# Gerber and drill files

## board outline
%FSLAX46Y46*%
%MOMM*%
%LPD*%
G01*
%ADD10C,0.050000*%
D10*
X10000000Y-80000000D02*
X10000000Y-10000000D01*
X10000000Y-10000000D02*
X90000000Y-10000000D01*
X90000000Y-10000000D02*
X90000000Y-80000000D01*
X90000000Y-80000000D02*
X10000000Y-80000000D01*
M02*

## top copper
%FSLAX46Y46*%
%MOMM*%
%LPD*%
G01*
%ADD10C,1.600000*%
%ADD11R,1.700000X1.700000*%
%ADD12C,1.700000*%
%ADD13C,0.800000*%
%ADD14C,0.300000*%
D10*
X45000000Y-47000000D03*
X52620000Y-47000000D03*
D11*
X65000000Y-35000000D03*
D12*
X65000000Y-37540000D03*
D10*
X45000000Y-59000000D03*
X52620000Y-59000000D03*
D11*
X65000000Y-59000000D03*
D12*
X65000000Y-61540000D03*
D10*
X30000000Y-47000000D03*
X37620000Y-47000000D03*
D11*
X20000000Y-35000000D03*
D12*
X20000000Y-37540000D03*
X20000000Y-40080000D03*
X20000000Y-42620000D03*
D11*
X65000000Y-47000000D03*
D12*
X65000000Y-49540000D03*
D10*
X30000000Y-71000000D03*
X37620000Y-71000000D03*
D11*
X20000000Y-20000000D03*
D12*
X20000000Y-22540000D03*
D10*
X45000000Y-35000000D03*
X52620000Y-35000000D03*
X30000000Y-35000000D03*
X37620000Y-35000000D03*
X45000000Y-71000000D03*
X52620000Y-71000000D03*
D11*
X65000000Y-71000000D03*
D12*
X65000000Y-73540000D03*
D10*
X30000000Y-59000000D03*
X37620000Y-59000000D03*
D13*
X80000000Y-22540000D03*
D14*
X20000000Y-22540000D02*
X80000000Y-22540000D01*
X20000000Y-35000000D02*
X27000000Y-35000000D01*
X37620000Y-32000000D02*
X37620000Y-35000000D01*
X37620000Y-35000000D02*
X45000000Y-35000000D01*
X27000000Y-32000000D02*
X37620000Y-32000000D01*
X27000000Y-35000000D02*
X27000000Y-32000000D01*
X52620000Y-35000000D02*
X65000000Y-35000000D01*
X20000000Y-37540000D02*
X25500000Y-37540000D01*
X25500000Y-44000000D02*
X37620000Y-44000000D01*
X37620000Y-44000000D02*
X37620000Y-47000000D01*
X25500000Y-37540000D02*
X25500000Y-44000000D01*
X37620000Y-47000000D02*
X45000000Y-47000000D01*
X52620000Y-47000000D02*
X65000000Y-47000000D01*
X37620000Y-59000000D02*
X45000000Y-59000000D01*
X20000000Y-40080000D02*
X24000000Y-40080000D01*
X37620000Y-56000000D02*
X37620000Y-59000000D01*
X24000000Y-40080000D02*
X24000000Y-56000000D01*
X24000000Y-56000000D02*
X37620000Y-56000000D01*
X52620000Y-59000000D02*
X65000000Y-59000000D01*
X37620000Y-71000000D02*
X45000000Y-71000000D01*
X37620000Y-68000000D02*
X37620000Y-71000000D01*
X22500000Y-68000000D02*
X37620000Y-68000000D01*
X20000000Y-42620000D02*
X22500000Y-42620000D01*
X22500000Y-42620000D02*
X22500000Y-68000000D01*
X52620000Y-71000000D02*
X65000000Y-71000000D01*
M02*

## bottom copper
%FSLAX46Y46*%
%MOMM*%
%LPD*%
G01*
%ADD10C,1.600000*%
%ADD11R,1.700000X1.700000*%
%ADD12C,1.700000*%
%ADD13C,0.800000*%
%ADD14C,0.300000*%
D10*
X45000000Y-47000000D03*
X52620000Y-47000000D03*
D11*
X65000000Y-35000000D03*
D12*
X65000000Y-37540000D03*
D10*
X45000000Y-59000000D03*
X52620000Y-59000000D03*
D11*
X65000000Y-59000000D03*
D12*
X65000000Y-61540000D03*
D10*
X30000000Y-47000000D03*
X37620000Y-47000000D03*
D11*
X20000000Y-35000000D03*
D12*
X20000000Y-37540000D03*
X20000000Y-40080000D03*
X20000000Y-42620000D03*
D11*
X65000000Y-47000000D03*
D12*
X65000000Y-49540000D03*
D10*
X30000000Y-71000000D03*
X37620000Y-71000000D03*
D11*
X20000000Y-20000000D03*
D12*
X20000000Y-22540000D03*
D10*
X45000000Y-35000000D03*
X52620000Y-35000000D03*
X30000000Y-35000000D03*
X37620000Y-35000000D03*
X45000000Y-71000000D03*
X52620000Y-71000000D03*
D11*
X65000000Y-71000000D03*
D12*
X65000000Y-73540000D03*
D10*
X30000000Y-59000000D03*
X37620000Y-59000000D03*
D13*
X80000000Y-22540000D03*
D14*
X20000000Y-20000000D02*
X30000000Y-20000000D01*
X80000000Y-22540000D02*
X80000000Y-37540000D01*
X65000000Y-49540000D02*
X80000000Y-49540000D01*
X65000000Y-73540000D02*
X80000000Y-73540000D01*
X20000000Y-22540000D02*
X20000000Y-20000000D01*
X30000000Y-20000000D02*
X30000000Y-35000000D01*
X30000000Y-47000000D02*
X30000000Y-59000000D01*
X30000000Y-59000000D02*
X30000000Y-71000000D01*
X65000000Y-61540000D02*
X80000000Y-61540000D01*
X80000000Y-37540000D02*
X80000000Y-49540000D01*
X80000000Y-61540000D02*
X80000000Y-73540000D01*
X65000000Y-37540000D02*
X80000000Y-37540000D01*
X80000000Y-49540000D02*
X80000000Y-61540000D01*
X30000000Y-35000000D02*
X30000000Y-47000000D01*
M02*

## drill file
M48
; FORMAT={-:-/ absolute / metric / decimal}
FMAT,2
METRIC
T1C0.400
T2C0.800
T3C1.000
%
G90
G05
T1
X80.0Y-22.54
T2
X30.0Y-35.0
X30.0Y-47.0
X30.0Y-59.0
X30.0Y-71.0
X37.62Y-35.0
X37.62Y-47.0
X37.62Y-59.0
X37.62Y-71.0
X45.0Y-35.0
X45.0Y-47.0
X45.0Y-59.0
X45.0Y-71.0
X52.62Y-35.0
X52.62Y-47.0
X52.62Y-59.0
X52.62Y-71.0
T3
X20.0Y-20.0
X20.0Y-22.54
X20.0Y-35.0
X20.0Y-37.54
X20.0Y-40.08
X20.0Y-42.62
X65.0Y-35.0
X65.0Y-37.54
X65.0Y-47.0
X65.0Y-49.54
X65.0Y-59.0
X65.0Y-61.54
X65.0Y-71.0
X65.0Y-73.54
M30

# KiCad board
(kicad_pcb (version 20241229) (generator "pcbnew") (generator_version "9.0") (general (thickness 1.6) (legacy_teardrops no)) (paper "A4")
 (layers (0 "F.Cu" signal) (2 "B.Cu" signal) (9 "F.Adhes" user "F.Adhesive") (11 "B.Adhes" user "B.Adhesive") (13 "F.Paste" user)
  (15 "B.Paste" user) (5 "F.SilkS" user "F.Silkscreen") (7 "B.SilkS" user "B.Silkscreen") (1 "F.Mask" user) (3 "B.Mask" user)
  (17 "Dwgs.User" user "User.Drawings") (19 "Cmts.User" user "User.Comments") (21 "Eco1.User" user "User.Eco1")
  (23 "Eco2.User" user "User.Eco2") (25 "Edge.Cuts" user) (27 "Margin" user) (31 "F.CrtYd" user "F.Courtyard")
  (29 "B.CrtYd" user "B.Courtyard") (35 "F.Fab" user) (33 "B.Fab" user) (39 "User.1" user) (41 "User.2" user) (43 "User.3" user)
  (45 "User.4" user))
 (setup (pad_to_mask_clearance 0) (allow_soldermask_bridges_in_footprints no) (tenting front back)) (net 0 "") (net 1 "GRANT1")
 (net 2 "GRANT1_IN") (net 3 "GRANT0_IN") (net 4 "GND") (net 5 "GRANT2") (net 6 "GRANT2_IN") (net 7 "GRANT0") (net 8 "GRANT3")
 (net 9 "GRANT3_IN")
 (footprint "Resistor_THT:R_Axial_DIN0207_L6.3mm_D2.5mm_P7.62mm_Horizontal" (layer "F.Cu") (at 45 47)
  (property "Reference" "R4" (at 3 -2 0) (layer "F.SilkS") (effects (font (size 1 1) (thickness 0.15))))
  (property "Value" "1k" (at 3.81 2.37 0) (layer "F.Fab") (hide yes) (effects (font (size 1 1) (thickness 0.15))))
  (pad "1" thru_hole circle (at 0 0) (size 1.6 1.6) (drill 0.8) (layers "*.Cu" "*.Mask") (remove_unused_layers no) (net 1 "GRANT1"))
  (pad "2" thru_hole circle (at 7.62 0) (size 1.6 1.6) (drill 0.8) (layers "*.Cu" "*.Mask") (remove_unused_layers no) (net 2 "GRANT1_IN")))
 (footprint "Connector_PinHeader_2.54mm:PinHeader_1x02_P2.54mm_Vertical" (layer "F.Cu") (at 65 35)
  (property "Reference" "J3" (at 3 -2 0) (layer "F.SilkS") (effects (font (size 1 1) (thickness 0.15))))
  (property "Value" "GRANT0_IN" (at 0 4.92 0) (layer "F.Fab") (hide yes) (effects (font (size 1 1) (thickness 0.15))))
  (pad "1" thru_hole rect (at 0 0) (size 1.7 1.7) (drill 1) (layers "*.Cu" "*.Mask") (remove_unused_layers no) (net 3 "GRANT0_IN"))
  (pad "2" thru_hole circle (at 0 2.54) (size 1.7 1.7) (drill 1) (layers "*.Cu" "*.Mask") (remove_unused_layers no) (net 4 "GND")))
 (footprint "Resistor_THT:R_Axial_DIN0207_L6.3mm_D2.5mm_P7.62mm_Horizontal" (layer "F.Cu") (at 45 59)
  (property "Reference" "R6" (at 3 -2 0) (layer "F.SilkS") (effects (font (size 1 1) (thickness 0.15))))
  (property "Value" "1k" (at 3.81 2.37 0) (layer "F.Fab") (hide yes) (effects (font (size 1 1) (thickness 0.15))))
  (pad "1" thru_hole circle (at 0 0) (size 1.6 1.6) (drill 0.8) (layers "*.Cu" "*.Mask") (remove_unused_layers no) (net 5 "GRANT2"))
  (pad "2" thru_hole circle (at 7.62 0) (size 1.6 1.6) (drill 0.8) (layers "*.Cu" "*.Mask") (remove_unused_layers no) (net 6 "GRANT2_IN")))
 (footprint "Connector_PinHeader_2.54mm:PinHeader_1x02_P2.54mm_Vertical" (layer "F.Cu") (at 65 59)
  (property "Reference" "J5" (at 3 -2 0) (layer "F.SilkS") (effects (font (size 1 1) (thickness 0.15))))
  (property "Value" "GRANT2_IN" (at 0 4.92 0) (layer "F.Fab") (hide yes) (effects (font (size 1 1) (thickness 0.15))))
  (pad "1" thru_hole rect (at 0 0) (size 1.7 1.7) (drill 1) (layers "*.Cu" "*.Mask") (remove_unused_layers no) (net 6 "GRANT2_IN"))
  (pad "2" thru_hole circle (at 0 2.54) (size 1.7 1.7) (drill 1) (layers "*.Cu" "*.Mask") (remove_unused_layers no) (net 4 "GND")))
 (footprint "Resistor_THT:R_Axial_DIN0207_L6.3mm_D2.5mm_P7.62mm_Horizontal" (layer "F.Cu") (at 30 47)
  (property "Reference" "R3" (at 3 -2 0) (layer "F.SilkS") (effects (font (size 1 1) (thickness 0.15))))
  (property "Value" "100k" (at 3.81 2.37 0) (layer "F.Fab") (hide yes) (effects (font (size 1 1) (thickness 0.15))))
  (pad "1" thru_hole circle (at 0 0) (size 1.6 1.6) (drill 0.8) (layers "*.Cu" "*.Mask") (remove_unused_layers no) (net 4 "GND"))
  (pad "2" thru_hole circle (at 7.62 0) (size 1.6 1.6) (drill 0.8) (layers "*.Cu" "*.Mask") (remove_unused_layers no) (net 1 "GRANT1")))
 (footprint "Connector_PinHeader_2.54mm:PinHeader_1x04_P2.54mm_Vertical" (layer "F.Cu") (at 20 35)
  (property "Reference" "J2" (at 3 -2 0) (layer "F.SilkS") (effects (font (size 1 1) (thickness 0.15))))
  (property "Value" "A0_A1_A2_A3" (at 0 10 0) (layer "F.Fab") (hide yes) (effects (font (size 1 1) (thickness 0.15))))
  (pad "1" thru_hole rect (at 0 0) (size 1.7 1.7) (drill 1) (layers "*.Cu" "*.Mask") (remove_unused_layers no) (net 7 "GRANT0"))
  (pad "2" thru_hole circle (at 0 2.54) (size 1.7 1.7) (drill 1) (layers "*.Cu" "*.Mask") (remove_unused_layers no) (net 1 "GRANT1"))
  (pad "3" thru_hole circle (at 0 5.08) (size 1.7 1.7) (drill 1) (layers "*.Cu" "*.Mask") (remove_unused_layers no) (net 5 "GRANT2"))
  (pad "4" thru_hole circle (at 0 7.62) (size 1.7 1.7) (drill 1) (layers "*.Cu" "*.Mask") (remove_unused_layers no) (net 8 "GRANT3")))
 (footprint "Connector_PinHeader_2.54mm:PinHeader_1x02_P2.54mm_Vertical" (layer "F.Cu") (at 65 47)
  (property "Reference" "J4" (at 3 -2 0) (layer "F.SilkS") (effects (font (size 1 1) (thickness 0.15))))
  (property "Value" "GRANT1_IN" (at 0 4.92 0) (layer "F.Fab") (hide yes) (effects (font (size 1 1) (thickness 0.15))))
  (pad "1" thru_hole rect (at 0 0) (size 1.7 1.7) (drill 1) (layers "*.Cu" "*.Mask") (remove_unused_layers no) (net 2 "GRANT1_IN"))
  (pad "2" thru_hole circle (at 0 2.54) (size 1.7 1.7) (drill 1) (layers "*.Cu" "*.Mask") (remove_unused_layers no) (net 4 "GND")))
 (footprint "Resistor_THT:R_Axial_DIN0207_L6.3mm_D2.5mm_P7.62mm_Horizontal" (layer "F.Cu") (at 30 71)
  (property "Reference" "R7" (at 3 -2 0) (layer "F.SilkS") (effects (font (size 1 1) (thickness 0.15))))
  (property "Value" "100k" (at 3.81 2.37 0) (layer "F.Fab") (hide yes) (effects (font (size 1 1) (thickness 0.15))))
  (pad "1" thru_hole circle (at 0 0) (size 1.6 1.6) (drill 0.8) (layers "*.Cu" "*.Mask") (remove_unused_layers no) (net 4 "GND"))
  (pad "2" thru_hole circle (at 7.62 0) (size 1.6 1.6) (drill 0.8) (layers "*.Cu" "*.Mask") (remove_unused_layers no) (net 8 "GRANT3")))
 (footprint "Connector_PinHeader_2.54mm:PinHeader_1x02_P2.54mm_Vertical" (layer "F.Cu") (at 20 20)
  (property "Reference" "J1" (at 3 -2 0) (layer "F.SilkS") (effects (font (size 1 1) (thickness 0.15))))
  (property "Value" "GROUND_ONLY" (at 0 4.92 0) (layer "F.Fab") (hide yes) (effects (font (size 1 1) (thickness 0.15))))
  (pad "1" thru_hole rect (at 0 0) (size 1.7 1.7) (drill 1) (layers "*.Cu" "*.Mask") (remove_unused_layers no) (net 4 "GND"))
  (pad "2" thru_hole circle (at 0 2.54) (size 1.7 1.7) (drill 1) (layers "*.Cu" "*.Mask") (remove_unused_layers no) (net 4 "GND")))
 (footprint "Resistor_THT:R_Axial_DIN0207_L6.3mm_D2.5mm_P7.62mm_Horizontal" (layer "F.Cu") (at 45 35)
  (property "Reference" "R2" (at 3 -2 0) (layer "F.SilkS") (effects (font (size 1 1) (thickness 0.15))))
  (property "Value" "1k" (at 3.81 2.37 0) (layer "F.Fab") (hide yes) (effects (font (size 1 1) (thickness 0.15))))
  (pad "1" thru_hole circle (at 0 0) (size 1.6 1.6) (drill 0.8) (layers "*.Cu" "*.Mask") (remove_unused_layers no) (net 7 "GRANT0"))
  (pad "2" thru_hole circle (at 7.62 0) (size 1.6 1.6) (drill 0.8) (layers "*.Cu" "*.Mask") (remove_unused_layers no) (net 3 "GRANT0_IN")))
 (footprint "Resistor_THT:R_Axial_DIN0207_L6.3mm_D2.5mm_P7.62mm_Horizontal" (layer "F.Cu") (at 30 35)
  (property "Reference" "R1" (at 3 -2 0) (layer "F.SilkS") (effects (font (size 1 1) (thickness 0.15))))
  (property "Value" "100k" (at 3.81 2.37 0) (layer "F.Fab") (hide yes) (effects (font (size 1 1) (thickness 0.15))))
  (pad "1" thru_hole circle (at 0 0) (size 1.6 1.6) (drill 0.8) (layers "*.Cu" "*.Mask") (remove_unused_layers no) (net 4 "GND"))
  (pad "2" thru_hole circle (at 7.62 0) (size 1.6 1.6) (drill 0.8) (layers "*.Cu" "*.Mask") (remove_unused_layers no) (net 7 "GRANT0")))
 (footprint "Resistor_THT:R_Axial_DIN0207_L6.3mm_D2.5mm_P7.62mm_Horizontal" (layer "F.Cu") (at 45 71)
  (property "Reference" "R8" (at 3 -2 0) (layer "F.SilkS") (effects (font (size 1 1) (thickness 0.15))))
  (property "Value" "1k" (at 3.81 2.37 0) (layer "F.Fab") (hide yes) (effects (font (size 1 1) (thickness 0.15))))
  (pad "1" thru_hole circle (at 0 0) (size 1.6 1.6) (drill 0.8) (layers "*.Cu" "*.Mask") (remove_unused_layers no) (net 8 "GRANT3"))
  (pad "2" thru_hole circle (at 7.62 0) (size 1.6 1.6) (drill 0.8) (layers "*.Cu" "*.Mask") (remove_unused_layers no) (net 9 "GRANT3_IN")))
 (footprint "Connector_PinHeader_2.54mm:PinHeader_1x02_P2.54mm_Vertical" (layer "F.Cu") (at 65 71)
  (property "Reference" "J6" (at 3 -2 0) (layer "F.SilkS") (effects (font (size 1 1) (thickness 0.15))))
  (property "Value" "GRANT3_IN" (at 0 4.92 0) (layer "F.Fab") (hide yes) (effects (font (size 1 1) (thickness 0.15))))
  (pad "1" thru_hole rect (at 0 0) (size 1.7 1.7) (drill 1) (layers "*.Cu" "*.Mask") (remove_unused_layers no) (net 9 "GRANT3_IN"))
  (pad "2" thru_hole circle (at 0 2.54) (size 1.7 1.7) (drill 1) (layers "*.Cu" "*.Mask") (remove_unused_layers no) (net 4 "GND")))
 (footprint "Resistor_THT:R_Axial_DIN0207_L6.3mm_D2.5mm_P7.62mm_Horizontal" (layer "F.Cu") (at 30 59)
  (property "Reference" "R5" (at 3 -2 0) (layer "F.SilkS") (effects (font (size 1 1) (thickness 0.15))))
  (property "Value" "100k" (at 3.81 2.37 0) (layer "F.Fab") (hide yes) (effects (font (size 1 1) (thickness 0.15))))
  (pad "1" thru_hole circle (at 0 0) (size 1.6 1.6) (drill 0.8) (layers "*.Cu" "*.Mask") (remove_unused_layers no) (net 4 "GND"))
  (pad "2" thru_hole circle (at 7.62 0) (size 1.6 1.6) (drill 0.8) (layers "*.Cu" "*.Mask") (remove_unused_layers no) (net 5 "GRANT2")))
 (gr_line (start 10 80) (end 10 10) (stroke (width 0.05) (type default)) (layer "Edge.Cuts"))
 (gr_line (start 10 10) (end 90 10) (stroke (width 0.05) (type default)) (layer "Edge.Cuts"))
 (gr_line (start 90 10) (end 90 80) (stroke (width 0.05) (type default)) (layer "Edge.Cuts"))
 (gr_line (start 90 80) (end 10 80) (stroke (width 0.05) (type default)) (layer "Edge.Cuts"))
 (segment (start 20 22.54) (end 80 22.54) (width 0.3) (layer "F.Cu") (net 4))
 (via (at 80 22.54) (size 0.8) (drill 0.4) (layers "F.Cu" "B.Cu") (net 4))
 (segment (start 20 20) (end 30 20) (width 0.3) (layer "B.Cu") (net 4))
 (segment (start 80 22.54) (end 80 37.54) (width 0.3) (layer "B.Cu") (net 4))
 (segment (start 65 49.54) (end 80 49.54) (width 0.3) (layer "B.Cu") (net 4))
 (segment (start 65 73.54) (end 80 73.54) (width 0.3) (layer "B.Cu") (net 4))
 (segment (start 20 22.54) (end 20 20) (width 0.3) (layer "B.Cu") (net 4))
 (segment (start 30 20) (end 30 35) (width 0.3) (layer "B.Cu") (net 4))
 (segment (start 30 47) (end 30 59) (width 0.3) (layer "B.Cu") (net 4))
 (segment (start 30 59) (end 30 71) (width 0.3) (layer "B.Cu") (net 4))
 (segment (start 65 61.54) (end 80 61.54) (width 0.3) (layer "B.Cu") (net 4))
 (segment (start 80 37.54) (end 80 49.54) (width 0.3) (layer "B.Cu") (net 4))
 (segment (start 80 61.54) (end 80 73.54) (width 0.3) (layer "B.Cu") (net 4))
 (segment (start 65 37.54) (end 80 37.54) (width 0.3) (layer "B.Cu") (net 4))
 (segment (start 80 49.54) (end 80 61.54) (width 0.3) (layer "B.Cu") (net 4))
 (segment (start 30 35) (end 30 47) (width 0.3) (layer "B.Cu") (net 4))
 (segment (start 20 35) (end 27 35) (width 0.3) (layer "F.Cu") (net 7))
 (segment (start 37.62 32) (end 37.62 35) (width 0.3) (layer "F.Cu") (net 7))
 (segment (start 37.62 35) (end 45 35) (width 0.3) (layer "F.Cu") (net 7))
 (segment (start 27 32) (end 37.62 32) (width 0.3) (layer "F.Cu") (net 7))
 (segment (start 27 35) (end 27 32) (width 0.3) (layer "F.Cu") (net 7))
 (segment (start 52.62 35) (end 65 35) (width 0.3) (layer "F.Cu") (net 3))
 (segment (start 20 37.54) (end 25.5 37.54) (width 0.3) (layer "F.Cu") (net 1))
 (segment (start 25.5 44) (end 37.62 44) (width 0.3) (layer "F.Cu") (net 1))
 (segment (start 37.62 44) (end 37.62 47) (width 0.3) (layer "F.Cu") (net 1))
 (segment (start 25.5 37.54) (end 25.5 44) (width 0.3) (layer "F.Cu") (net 1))
 (segment (start 37.62 47) (end 45 47) (width 0.3) (layer "F.Cu") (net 1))
 (segment (start 52.62 47) (end 65 47) (width 0.3) (layer "F.Cu") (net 2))
 (segment (start 37.62 59) (end 45 59) (width 0.3) (layer "F.Cu") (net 5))
 (segment (start 20 40.08) (end 24 40.08) (width 0.3) (layer "F.Cu") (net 5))
 (segment (start 37.62 56) (end 37.62 59) (width 0.3) (layer "F.Cu") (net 5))
 (segment (start 24 40.08) (end 24 56) (width 0.3) (layer "F.Cu") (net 5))
 (segment (start 24 56) (end 37.62 56) (width 0.3) (layer "F.Cu") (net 5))
 (segment (start 52.62 59) (end 65 59) (width 0.3) (layer "F.Cu") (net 6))
 (segment (start 37.62 71) (end 45 71) (width 0.3) (layer "F.Cu") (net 8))
 (segment (start 37.62 68) (end 37.62 71) (width 0.3) (layer "F.Cu") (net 8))
 (segment (start 22.5 68) (end 37.62 68) (width 0.3) (layer "F.Cu") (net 8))
 (segment (start 20 42.62) (end 22.5 42.62) (width 0.3) (layer "F.Cu") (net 8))
 (segment (start 22.5 42.62) (end 22.5 68) (width 0.3) (layer "F.Cu") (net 8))
 (segment (start 52.62 71) (end 65 71) (width 0.3) (layer "F.Cu") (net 9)))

